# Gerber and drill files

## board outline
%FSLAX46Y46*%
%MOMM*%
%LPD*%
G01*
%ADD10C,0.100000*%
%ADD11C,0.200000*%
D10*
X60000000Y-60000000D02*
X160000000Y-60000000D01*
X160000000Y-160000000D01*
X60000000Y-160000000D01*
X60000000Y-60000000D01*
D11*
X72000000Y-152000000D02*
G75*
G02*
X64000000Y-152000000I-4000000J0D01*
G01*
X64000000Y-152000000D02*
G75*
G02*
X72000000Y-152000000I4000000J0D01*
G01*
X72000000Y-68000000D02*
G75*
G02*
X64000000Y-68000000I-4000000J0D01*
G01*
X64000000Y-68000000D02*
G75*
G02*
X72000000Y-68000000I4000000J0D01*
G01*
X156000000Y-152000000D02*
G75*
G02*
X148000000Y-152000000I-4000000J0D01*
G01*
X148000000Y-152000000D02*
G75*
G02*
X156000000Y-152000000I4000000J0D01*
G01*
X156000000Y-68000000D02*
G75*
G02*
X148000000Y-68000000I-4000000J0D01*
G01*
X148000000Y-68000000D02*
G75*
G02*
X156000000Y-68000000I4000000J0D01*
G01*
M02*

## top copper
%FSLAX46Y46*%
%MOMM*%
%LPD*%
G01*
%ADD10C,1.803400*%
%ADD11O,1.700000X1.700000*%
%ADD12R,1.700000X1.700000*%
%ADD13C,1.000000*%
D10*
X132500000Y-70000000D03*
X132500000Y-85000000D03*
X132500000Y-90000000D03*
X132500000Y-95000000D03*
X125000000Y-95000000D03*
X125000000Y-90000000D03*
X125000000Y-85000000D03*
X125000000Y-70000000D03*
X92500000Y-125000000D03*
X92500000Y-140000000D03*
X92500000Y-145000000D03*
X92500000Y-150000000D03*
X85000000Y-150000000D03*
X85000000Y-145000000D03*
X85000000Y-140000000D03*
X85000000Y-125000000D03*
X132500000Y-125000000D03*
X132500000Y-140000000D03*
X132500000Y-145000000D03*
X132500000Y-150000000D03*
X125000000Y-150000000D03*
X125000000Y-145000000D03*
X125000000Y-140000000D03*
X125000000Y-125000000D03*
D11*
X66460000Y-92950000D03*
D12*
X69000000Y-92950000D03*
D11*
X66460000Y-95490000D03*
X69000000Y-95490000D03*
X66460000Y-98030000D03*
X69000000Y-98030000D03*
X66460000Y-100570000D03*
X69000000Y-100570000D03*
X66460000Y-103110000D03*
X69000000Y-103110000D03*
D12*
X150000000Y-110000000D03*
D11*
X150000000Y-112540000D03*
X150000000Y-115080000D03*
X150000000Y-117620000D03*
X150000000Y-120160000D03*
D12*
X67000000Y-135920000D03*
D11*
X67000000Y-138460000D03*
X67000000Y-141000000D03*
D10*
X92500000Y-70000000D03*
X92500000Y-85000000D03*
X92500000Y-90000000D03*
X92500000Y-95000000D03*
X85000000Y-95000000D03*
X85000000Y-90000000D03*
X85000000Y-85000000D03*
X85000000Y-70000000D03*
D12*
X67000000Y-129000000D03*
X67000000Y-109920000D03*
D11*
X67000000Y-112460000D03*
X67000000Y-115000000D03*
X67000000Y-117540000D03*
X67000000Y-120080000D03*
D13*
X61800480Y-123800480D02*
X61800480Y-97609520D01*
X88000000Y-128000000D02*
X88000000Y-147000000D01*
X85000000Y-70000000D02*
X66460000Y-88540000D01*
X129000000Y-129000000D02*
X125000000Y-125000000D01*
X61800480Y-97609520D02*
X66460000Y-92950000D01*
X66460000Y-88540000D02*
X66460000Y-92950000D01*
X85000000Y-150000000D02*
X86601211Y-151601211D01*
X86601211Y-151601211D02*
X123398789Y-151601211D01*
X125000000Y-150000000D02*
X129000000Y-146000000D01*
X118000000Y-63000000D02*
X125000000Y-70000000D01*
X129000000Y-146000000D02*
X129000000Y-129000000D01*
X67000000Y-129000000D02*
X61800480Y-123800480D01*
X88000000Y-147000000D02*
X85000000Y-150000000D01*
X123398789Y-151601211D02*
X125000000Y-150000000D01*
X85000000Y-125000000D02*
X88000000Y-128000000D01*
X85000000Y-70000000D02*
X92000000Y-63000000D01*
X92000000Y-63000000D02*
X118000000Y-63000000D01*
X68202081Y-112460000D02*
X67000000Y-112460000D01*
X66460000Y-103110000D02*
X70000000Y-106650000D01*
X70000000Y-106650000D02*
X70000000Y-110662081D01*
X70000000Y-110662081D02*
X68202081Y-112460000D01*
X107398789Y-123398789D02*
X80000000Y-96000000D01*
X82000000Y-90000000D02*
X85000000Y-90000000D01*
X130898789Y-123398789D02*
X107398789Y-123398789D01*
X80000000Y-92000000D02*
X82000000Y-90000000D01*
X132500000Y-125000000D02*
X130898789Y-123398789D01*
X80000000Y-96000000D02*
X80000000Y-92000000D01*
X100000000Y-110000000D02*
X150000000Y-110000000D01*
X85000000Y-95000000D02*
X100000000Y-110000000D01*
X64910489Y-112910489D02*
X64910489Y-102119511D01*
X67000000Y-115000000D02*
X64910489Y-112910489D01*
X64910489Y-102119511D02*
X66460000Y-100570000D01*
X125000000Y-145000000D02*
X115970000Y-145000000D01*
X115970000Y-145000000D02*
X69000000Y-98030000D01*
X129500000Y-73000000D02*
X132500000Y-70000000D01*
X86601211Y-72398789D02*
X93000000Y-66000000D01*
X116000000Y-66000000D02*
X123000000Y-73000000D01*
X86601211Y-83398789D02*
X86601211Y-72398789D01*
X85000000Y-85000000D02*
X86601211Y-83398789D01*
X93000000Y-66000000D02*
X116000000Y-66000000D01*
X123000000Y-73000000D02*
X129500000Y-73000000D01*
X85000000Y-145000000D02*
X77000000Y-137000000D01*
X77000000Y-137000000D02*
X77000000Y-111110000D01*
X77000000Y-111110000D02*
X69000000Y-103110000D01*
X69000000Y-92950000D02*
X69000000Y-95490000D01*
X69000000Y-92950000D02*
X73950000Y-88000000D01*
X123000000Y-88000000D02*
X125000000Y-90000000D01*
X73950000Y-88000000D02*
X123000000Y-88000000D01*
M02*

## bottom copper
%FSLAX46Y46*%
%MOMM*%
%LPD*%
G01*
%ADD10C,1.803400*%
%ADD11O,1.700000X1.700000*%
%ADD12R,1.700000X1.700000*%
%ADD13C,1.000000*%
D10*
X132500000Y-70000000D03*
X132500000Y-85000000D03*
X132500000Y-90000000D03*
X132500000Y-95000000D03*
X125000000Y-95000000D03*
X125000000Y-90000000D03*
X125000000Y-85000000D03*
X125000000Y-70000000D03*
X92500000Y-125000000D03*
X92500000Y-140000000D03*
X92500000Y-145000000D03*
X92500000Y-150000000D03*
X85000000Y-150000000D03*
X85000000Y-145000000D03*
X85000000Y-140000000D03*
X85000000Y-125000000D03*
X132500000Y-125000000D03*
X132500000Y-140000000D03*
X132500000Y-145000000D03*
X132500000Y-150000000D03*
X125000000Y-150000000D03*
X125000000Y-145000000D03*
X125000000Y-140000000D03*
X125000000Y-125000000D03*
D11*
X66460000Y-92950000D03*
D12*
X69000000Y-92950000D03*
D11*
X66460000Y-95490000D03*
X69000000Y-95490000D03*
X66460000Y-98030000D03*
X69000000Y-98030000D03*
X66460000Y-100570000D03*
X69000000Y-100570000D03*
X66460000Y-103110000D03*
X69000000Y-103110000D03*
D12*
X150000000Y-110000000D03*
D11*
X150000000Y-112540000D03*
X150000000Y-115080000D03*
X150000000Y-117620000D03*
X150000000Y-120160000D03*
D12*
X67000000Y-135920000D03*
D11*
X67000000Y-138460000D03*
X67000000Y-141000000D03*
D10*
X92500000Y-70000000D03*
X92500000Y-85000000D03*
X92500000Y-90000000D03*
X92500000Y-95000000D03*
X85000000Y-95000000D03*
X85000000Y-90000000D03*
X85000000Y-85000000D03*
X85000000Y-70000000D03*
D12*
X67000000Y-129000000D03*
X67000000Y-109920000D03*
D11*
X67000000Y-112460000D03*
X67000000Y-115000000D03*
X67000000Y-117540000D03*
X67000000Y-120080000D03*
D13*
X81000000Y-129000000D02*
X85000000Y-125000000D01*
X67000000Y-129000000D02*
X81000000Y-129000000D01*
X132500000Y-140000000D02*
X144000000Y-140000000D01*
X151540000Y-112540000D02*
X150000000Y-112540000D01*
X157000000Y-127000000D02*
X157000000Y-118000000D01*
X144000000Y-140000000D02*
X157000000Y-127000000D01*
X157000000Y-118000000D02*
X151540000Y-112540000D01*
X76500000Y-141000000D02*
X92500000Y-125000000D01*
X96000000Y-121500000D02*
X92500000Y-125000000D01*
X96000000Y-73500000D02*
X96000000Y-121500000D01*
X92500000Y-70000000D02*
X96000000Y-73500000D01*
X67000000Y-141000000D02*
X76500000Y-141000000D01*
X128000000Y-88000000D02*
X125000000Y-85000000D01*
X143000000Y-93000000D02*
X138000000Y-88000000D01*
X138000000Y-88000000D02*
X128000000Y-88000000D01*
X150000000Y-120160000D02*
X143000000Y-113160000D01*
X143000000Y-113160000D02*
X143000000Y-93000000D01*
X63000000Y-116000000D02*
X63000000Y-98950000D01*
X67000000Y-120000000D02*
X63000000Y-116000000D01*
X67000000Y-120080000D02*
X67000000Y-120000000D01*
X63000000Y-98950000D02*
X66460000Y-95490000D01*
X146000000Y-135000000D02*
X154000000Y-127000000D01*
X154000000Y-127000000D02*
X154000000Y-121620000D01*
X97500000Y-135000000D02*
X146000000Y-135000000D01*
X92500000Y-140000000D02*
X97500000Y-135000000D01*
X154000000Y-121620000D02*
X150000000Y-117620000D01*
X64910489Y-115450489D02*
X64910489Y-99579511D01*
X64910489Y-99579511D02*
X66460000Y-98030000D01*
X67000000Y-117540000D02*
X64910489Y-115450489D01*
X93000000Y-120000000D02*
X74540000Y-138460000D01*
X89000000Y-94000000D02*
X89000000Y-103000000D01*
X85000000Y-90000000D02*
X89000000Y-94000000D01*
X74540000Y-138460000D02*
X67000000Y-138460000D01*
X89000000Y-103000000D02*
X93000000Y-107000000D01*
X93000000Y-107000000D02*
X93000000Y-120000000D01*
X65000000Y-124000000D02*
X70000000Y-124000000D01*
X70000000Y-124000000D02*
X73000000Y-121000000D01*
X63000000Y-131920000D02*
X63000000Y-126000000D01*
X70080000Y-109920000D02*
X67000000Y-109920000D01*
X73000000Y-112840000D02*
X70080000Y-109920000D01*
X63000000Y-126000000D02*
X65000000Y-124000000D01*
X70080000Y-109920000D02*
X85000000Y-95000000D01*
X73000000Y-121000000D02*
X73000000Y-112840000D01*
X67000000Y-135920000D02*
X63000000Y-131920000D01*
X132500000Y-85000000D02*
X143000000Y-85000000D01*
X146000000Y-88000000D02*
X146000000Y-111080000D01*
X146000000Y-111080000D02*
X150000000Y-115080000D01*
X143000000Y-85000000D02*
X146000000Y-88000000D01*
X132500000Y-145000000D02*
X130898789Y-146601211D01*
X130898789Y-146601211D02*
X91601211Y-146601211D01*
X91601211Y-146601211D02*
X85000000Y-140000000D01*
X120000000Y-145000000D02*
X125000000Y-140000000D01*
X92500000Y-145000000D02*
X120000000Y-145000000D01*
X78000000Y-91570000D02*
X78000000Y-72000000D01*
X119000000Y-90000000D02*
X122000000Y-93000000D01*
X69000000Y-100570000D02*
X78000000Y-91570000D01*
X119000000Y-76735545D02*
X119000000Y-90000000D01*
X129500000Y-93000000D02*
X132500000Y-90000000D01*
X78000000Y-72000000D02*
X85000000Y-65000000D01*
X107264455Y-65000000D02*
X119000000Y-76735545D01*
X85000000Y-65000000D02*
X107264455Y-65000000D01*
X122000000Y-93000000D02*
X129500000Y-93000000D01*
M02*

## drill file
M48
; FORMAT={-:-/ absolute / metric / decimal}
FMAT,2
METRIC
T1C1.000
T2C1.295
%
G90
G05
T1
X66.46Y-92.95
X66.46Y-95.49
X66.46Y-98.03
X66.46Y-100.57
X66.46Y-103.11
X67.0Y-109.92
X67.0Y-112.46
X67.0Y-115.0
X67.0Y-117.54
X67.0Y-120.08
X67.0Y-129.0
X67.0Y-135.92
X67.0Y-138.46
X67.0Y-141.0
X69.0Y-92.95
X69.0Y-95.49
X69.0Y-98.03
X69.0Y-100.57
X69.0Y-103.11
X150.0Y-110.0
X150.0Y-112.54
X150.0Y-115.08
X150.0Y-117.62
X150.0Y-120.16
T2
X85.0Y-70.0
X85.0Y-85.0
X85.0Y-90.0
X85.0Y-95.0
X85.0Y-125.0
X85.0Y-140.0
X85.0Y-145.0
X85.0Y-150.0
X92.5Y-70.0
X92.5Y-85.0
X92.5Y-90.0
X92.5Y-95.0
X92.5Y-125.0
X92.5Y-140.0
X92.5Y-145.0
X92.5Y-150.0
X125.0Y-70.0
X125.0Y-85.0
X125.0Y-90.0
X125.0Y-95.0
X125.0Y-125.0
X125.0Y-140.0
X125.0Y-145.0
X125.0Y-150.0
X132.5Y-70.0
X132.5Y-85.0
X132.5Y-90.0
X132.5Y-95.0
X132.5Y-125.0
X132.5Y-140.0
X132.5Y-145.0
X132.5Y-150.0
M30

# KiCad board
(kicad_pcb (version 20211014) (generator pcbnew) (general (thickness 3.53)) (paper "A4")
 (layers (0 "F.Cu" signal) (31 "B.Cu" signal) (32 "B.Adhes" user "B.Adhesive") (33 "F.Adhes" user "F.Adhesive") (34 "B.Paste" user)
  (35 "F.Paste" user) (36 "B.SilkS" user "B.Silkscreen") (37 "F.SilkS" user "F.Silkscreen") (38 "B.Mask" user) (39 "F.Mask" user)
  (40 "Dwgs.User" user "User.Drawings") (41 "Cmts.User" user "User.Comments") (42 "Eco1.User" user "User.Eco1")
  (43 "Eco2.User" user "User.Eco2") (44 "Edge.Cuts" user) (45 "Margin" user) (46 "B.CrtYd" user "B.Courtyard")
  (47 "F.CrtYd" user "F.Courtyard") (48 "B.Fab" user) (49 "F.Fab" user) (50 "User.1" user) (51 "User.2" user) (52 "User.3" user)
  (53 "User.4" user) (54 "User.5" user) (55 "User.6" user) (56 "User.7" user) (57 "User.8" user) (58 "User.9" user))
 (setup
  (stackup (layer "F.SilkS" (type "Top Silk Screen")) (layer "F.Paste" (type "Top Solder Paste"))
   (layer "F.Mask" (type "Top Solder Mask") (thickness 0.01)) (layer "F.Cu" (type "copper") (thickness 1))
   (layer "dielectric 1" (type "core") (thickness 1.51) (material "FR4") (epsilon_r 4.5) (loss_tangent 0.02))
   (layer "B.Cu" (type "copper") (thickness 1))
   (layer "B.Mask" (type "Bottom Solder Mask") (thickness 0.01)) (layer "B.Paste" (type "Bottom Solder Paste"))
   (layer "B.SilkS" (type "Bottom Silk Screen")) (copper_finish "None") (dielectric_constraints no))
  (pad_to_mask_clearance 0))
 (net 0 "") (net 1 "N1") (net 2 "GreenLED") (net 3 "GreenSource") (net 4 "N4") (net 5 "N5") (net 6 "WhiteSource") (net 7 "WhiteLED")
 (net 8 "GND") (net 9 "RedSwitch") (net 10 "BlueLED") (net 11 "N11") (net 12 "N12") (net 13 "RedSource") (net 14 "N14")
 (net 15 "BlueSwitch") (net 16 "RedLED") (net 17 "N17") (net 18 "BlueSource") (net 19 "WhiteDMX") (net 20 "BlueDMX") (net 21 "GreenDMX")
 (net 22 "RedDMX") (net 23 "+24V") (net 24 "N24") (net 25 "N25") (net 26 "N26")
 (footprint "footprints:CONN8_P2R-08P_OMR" (layer "F.Cu") (at 125 70)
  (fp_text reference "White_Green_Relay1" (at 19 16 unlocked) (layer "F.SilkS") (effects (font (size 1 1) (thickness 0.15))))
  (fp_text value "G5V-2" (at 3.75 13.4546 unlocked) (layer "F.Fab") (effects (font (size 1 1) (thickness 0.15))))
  (pad "1" thru_hole circle (at 7.5 0) (size 1.8034 1.8034) (drill 1.2954) (layers *.Cu *.Mask) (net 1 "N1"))
  (pad "4" thru_hole circle (at 7.5 15) (size 1.8034 1.8034) (drill 1.2954) (layers *.Cu *.Mask) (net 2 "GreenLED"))
  (pad "6" thru_hole circle (at 7.5 20) (size 1.8034 1.8034) (drill 1.2954) (layers *.Cu *.Mask) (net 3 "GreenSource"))
  (pad "8" thru_hole circle (at 7.5 25) (size 1.8034 1.8034) (drill 1.2954) (layers *.Cu *.Mask) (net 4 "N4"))
  (pad "9" thru_hole circle (at 0 25) (size 1.8034 1.8034) (drill 1.2954) (layers *.Cu *.Mask) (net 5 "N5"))
  (pad "11" thru_hole circle (at 0 20) (size 1.8034 1.8034) (drill 1.2954) (layers *.Cu *.Mask) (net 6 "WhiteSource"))
  (pad "13" thru_hole circle (at 0 15) (size 1.8034 1.8034) (drill 1.2954) (layers *.Cu *.Mask) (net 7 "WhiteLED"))
  (pad "16" thru_hole circle (at 0 0) (size 1.8034 1.8034) (drill 1.2954) (layers *.Cu *.Mask) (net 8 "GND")))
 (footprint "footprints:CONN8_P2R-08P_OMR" (layer "F.Cu") (at 85 125)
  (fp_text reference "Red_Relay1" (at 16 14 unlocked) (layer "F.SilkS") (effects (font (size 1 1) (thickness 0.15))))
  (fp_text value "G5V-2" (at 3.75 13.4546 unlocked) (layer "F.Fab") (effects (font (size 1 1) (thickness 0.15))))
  (pad "1" thru_hole circle (at 7.5 0) (size 1.8034 1.8034) (drill 1.2954) (layers *.Cu *.Mask) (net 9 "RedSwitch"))
  (pad "4" thru_hole circle (at 7.5 15) (size 1.8034 1.8034) (drill 1.2954) (layers *.Cu *.Mask) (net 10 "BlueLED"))
  (pad "6" thru_hole circle (at 7.5 20) (size 1.8034 1.8034) (drill 1.2954) (layers *.Cu *.Mask) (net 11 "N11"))
  (pad "8" thru_hole circle (at 7.5 25) (size 1.8034 1.8034) (drill 1.2954) (layers *.Cu *.Mask) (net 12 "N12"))
  (pad "9" thru_hole circle (at 0 25) (size 1.8034 1.8034) (drill 1.2954) (layers *.Cu *.Mask) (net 8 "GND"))
  (pad "11" thru_hole circle (at 0 20) (size 1.8034 1.8034) (drill 1.2954) (layers *.Cu *.Mask) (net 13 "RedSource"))
  (pad "13" thru_hole circle (at 0 15) (size 1.8034 1.8034) (drill 1.2954) (layers *.Cu *.Mask) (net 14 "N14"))
  (pad "16" thru_hole circle (at 0 0) (size 1.8034 1.8034) (drill 1.2954) (layers *.Cu *.Mask) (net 8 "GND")))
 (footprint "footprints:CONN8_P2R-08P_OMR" (layer "F.Cu") (at 125 125)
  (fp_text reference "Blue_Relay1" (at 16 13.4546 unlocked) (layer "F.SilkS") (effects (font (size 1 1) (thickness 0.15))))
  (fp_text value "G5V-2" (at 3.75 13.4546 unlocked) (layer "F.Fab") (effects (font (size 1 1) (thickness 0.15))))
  (pad "1" thru_hole circle (at 7.5 0) (size 1.8034 1.8034) (drill 1.2954) (layers *.Cu *.Mask) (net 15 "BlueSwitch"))
  (pad "4" thru_hole circle (at 7.5 15) (size 1.8034 1.8034) (drill 1.2954) (layers *.Cu *.Mask) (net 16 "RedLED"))
  (pad "6" thru_hole circle (at 7.5 20) (size 1.8034 1.8034) (drill 1.2954) (layers *.Cu *.Mask) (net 14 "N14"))
  (pad "8" thru_hole circle (at 7.5 25) (size 1.8034 1.8034) (drill 1.2954) (layers *.Cu *.Mask) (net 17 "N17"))
  (pad "9" thru_hole circle (at 0 25) (size 1.8034 1.8034) (drill 1.2954) (layers *.Cu *.Mask) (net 8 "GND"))
  (pad "11" thru_hole circle (at 0 20) (size 1.8034 1.8034) (drill 1.2954) (layers *.Cu *.Mask) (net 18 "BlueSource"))
  (pad "13" thru_hole circle (at 0 15) (size 1.8034 1.8034) (drill 1.2954) (layers *.Cu *.Mask) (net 11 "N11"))
  (pad "16" thru_hole circle (at 0 0) (size 1.8034 1.8034) (drill 1.2954) (layers *.Cu *.Mask) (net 8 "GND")))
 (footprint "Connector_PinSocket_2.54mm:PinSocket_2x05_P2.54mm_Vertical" (layer "F.Cu") (at 69 92.95)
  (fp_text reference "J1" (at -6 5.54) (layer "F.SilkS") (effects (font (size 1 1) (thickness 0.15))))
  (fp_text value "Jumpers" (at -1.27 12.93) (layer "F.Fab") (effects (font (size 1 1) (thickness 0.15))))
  (pad "1a" thru_hole oval (at -2.54 0) (size 1.7 1.7) (drill 1) (layers *.Cu *.Mask) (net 8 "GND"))
  (pad "1b" thru_hole rect (at 0 0) (size 1.7 1.7) (drill 1) (layers *.Cu *.Mask) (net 6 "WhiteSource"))
  (pad "2a" thru_hole oval (at -2.54 2.54) (size 1.7 1.7) (drill 1) (layers *.Cu *.Mask) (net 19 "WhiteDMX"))
  (pad "2b" thru_hole oval (at 0 2.54) (size 1.7 1.7) (drill 1) (layers *.Cu *.Mask) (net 6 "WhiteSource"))
  (pad "3a" thru_hole oval (at -2.54 5.08) (size 1.7 1.7) (drill 1) (layers *.Cu *.Mask) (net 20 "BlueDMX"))
  (pad "3b" thru_hole oval (at 0 5.08) (size 1.7 1.7) (drill 1) (layers *.Cu *.Mask) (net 18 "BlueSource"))
  (pad "4a" thru_hole oval (at -2.54 7.62) (size 1.7 1.7) (drill 1) (layers *.Cu *.Mask) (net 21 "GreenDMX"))
  (pad "4b" thru_hole oval (at 0 7.62) (size 1.7 1.7) (drill 1) (layers *.Cu *.Mask) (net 3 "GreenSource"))
  (pad "5a" thru_hole oval (at -2.54 10.16) (size 1.7 1.7) (drill 1) (layers *.Cu *.Mask) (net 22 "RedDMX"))
  (pad "5b" thru_hole oval (at 0 10.16) (size 1.7 1.7) (drill 1) (layers *.Cu *.Mask) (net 13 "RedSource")))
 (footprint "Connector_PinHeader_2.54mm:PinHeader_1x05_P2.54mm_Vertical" (layer "F.Cu") (at 150 110)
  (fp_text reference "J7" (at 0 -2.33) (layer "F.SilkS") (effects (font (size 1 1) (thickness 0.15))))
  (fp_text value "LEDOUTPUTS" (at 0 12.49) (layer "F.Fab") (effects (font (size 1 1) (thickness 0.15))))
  (pad "1" thru_hole rect (at 0 0) (size 1.7 1.7) (drill 1) (layers *.Cu *.Mask) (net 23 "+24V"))
  (pad "2" thru_hole oval (at 0 2.54) (size 1.7 1.7) (drill 1) (layers *.Cu *.Mask) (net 16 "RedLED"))
  (pad "3" thru_hole oval (at 0 5.08) (size 1.7 1.7) (drill 1) (layers *.Cu *.Mask) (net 2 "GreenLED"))
  (pad "4" thru_hole oval (at 0 7.62) (size 1.7 1.7) (drill 1) (layers *.Cu *.Mask) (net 10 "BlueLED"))
  (pad "5" thru_hole oval (at 0 10.16) (size 1.7 1.7) (drill 1) (layers *.Cu *.Mask) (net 7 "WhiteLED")))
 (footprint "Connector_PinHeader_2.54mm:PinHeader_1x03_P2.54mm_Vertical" (layer "F.Cu") (at 67 135.92)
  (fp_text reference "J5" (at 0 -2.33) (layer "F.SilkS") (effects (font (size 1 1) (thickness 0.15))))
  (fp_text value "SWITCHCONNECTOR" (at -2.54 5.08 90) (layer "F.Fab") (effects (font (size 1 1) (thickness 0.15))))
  (pad "1" thru_hole rect (at 0 0) (size 1.7 1.7) (drill 1) (layers *.Cu *.Mask) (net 23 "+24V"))
  (pad "2" thru_hole oval (at 0 2.54) (size 1.7 1.7) (drill 1) (layers *.Cu *.Mask) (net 15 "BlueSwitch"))
  (pad "3" thru_hole oval (at 0 5.08) (size 1.7 1.7) (drill 1) (layers *.Cu *.Mask) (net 9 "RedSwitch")))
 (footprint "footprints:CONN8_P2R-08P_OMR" (layer "F.Cu") (at 85 70)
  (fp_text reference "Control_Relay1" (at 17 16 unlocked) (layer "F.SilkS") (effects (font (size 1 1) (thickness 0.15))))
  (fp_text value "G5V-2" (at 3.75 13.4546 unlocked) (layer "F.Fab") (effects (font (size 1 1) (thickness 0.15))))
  (pad "1" thru_hole circle (at 7.5 0) (size 1.8034 1.8034) (drill 1.2954) (layers *.Cu *.Mask) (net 9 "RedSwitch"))
  (pad "4" thru_hole circle (at 7.5 15) (size 1.8034 1.8034) (drill 1.2954) (layers *.Cu *.Mask) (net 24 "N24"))
  (pad "6" thru_hole circle (at 7.5 20) (size 1.8034 1.8034) (drill 1.2954) (layers *.Cu *.Mask) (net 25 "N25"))
  (pad "8" thru_hole circle (at 7.5 25) (size 1.8034 1.8034) (drill 1.2954) (layers *.Cu *.Mask) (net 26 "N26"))
  (pad "9" thru_hole circle (at 0 25) (size 1.8034 1.8034) (drill 1.2954) (layers *.Cu *.Mask) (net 23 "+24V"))
  (pad "11" thru_hole circle (at 0 20) (size 1.8034 1.8034) (drill 1.2954) (layers *.Cu *.Mask) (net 15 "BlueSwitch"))
  (pad "13" thru_hole circle (at 0 15) (size 1.8034 1.8034) (drill 1.2954) (layers *.Cu *.Mask) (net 1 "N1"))
  (pad "16" thru_hole circle (at 0 0) (size 1.8034 1.8034) (drill 1.2954) (layers *.Cu *.Mask) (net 8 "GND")))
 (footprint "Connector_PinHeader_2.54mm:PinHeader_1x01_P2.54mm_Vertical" (layer "F.Cu") (at 67 129)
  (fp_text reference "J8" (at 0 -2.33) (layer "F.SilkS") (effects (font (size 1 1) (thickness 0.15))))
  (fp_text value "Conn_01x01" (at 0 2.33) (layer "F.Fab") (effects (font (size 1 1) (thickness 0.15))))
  (pad "1" thru_hole rect (at 0 0) (size 1.7 1.7) (drill 1) (layers *.Cu *.Mask) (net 8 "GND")))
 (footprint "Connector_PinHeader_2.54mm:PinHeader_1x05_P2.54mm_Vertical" (layer "F.Cu") (at 67 109.92)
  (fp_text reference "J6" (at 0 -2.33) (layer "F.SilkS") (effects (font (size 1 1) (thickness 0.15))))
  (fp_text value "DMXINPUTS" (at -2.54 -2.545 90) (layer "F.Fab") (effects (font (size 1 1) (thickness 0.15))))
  (pad "1" thru_hole rect (at 0 0) (size 1.7 1.7) (drill 1) (layers *.Cu *.Mask) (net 23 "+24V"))
  (pad "2" thru_hole oval (at 0 2.54) (size 1.7 1.7) (drill 1) (layers *.Cu *.Mask) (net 22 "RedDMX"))
  (pad "3" thru_hole oval (at 0 5.08) (size 1.7 1.7) (drill 1) (layers *.Cu *.Mask) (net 21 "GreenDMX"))
  (pad "4" thru_hole oval (at 0 7.62) (size 1.7 1.7) (drill 1) (layers *.Cu *.Mask) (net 20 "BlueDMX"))
  (pad "5" thru_hole oval (at 0 10.16) (size 1.7 1.7) (drill 1) (layers *.Cu *.Mask) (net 19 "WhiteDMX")))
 (gr_rect (start 60 60) (end 160 160) (layer "Edge.Cuts") (width 0.1) (fill none))
 (gr_circle (center 68 152) (end 72 152) (layer "Edge.Cuts") (width 0.2) (fill none))
 (gr_circle (center 68 68) (end 72 68) (layer "Edge.Cuts") (width 0.2) (fill none))
 (gr_circle (center 152 152) (end 156 152) (layer "Edge.Cuts") (width 0.2) (fill none))
 (gr_circle (center 152 68) (end 156 68) (layer "Edge.Cuts") (width 0.2) (fill none))
 (segment (start 61.80048 123.80048) (end 61.80048 97.60952) (width 1) (layer "F.Cu") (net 8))
 (segment (start 88 128) (end 88 147) (width 1) (layer "F.Cu") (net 8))
 (segment (start 85 70) (end 66.46 88.54) (width 1) (layer "F.Cu") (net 8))
 (segment (start 129 129) (end 125 125) (width 1) (layer "F.Cu") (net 8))
 (segment (start 61.80048 97.60952) (end 66.46 92.95) (width 1) (layer "F.Cu") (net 8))
 (segment (start 66.46 88.54) (end 66.46 92.95) (width 1) (layer "F.Cu") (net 8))
 (segment (start 85 150) (end 86.601211 151.601211) (width 1) (layer "F.Cu") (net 8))
 (segment (start 86.601211 151.601211) (end 123.398789 151.601211) (width 1) (layer "F.Cu") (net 8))
 (segment (start 125 150) (end 129 146) (width 1) (layer "F.Cu") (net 8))
 (segment (start 118 63) (end 125 70) (width 1) (layer "F.Cu") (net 8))
 (segment (start 129 146) (end 129 129) (width 1) (layer "F.Cu") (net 8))
 (segment (start 67 129) (end 61.80048 123.80048) (width 1) (layer "F.Cu") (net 8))
 (segment (start 88 147) (end 85 150) (width 1) (layer "F.Cu") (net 8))
 (segment (start 123.398789 151.601211) (end 125 150) (width 1) (layer "F.Cu") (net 8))
 (segment (start 85 125) (end 88 128) (width 1) (layer "F.Cu") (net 8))
 (segment (start 85 70) (end 92 63) (width 1) (layer "F.Cu") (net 8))
 (segment (start 92 63) (end 118 63) (width 1) (layer "F.Cu") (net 8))
 (segment (start 81 129) (end 85 125) (width 1) (layer "B.Cu") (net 8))
 (segment (start 67 129) (end 81 129) (width 1) (layer "B.Cu") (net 8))
 (segment (start 132.5 140) (end 144 140) (width 1) (layer "B.Cu") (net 16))
 (segment (start 151.54 112.54) (end 150 112.54) (width 1) (layer "B.Cu") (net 16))
 (segment (start 157 127) (end 157 118) (width 1) (layer "B.Cu") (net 16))
 (segment (start 144 140) (end 157 127) (width 1) (layer "B.Cu") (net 16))
 (segment (start 157 118) (end 151.54 112.54) (width 1) (layer "B.Cu") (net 16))
 (segment (start 68.202081 112.46) (end 67 112.46) (width 1) (layer "F.Cu") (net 22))
 (segment (start 66.46 103.11) (end 70 106.65) (width 1) (layer "F.Cu") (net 22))
 (segment (start 70 106.65) (end 70 110.662081) (width 1) (layer "F.Cu") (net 22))
 (segment (start 70 110.662081) (end 68.202081 112.46) (width 1) (layer "F.Cu") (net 22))
 (segment (start 76.5 141) (end 92.5 125) (width 1) (layer "B.Cu") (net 9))
 (segment (start 96 121.5) (end 92.5 125) (width 1) (layer "B.Cu") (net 9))
 (segment (start 96 73.5) (end 96 121.5) (width 1) (layer "B.Cu") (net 9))
 (segment (start 92.5 70) (end 96 73.5) (width 1) (layer "B.Cu") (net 9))
 (segment (start 67 141) (end 76.5 141) (width 1) (layer "B.Cu") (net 9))
 (segment (start 128 88) (end 125 85) (width 1) (layer "B.Cu") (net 7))
 (segment (start 143 93) (end 138 88) (width 1) (layer "B.Cu") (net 7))
 (segment (start 138 88) (end 128 88) (width 1) (layer "B.Cu") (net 7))
 (segment (start 150 120.16) (end 143 113.16) (width 1) (layer "B.Cu") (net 7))
 (segment (start 143 113.16) (end 143 93) (width 1) (layer "B.Cu") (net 7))
 (segment (start 63 116) (end 63 98.95) (width 1) (layer "B.Cu") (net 19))
 (segment (start 67 120) (end 63 116) (width 1) (layer "B.Cu") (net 19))
 (segment (start 67 120.08) (end 67 120) (width 1) (layer "B.Cu") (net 19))
 (segment (start 63 98.95) (end 66.46 95.49) (width 1) (layer "B.Cu") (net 19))
 (segment (start 146 135) (end 154 127) (width 1) (layer "B.Cu") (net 10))
 (segment (start 154 127) (end 154 121.62) (width 1) (layer "B.Cu") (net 10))
 (segment (start 97.5 135) (end 146 135) (width 1) (layer "B.Cu") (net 10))
 (segment (start 92.5 140) (end 97.5 135) (width 1) (layer "B.Cu") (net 10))
 (segment (start 154 121.62) (end 150 117.62) (width 1) (layer "B.Cu") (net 10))
 (segment (start 64.910489 115.450489) (end 64.910489 99.579511) (width 1) (layer "B.Cu") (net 20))
 (segment (start 64.910489 99.579511) (end 66.46 98.03) (width 1) (layer "B.Cu") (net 20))
 (segment (start 67 117.54) (end 64.910489 115.450489) (width 1) (layer "B.Cu") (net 20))
 (segment (start 107.398789 123.398789) (end 80 96) (width 1) (layer "F.Cu") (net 15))
 (segment (start 82 90) (end 85 90) (width 1) (layer "F.Cu") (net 15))
 (segment (start 130.898789 123.398789) (end 107.398789 123.398789) (width 1) (layer "F.Cu") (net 15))
 (segment (start 80 92) (end 82 90) (width 1) (layer "F.Cu") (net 15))
 (segment (start 132.5 125) (end 130.898789 123.398789) (width 1) (layer "F.Cu") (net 15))
 (segment (start 80 96) (end 80 92) (width 1) (layer "F.Cu") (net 15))
 (segment (start 93 120) (end 74.54 138.46) (width 1) (layer "B.Cu") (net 15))
 (segment (start 89 94) (end 89 103) (width 1) (layer "B.Cu") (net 15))
 (segment (start 85 90) (end 89 94) (width 1) (layer "B.Cu") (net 15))
 (segment (start 74.54 138.46) (end 67 138.46) (width 1) (layer "B.Cu") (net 15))
 (segment (start 89 103) (end 93 107) (width 1) (layer "B.Cu") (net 15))
 (segment (start 93 107) (end 93 120) (width 1) (layer "B.Cu") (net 15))
 (segment (start 100 110) (end 150 110) (width 1) (layer "F.Cu") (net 23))
 (segment (start 85 95) (end 100 110) (width 1) (layer "F.Cu") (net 23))
 (segment (start 65 124) (end 70 124) (width 1) (layer "B.Cu") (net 23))
 (segment (start 70 124) (end 73 121) (width 1) (layer "B.Cu") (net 23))
 (segment (start 63 131.92) (end 63 126) (width 1) (layer "B.Cu") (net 23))
 (segment (start 70.08 109.92) (end 67 109.92) (width 1) (layer "B.Cu") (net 23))
 (segment (start 73 112.84) (end 70.08 109.92) (width 1) (layer "B.Cu") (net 23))
 (segment (start 63 126) (end 65 124) (width 1) (layer "B.Cu") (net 23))
 (segment (start 70.08 109.92) (end 85 95) (width 1) (layer "B.Cu") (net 23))
 (segment (start 73 121) (end 73 112.84) (width 1) (layer "B.Cu") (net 23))
 (segment (start 67 135.92) (end 63 131.92) (width 1) (layer "B.Cu") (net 23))
 (segment (start 64.910489 112.910489) (end 64.910489 102.119511) (width 1) (layer "F.Cu") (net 21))
 (segment (start 67 115) (end 64.910489 112.910489) (width 1) (layer "F.Cu") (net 21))
 (segment (start 64.910489 102.119511) (end 66.46 100.57) (width 1) (layer "F.Cu") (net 21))
 (segment (start 132.5 85) (end 143 85) (width 1) (layer "B.Cu") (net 2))
 (segment (start 146 88) (end 146 111.08) (width 1) (layer "B.Cu") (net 2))
 (segment (start 146 111.08) (end 150 115.08) (width 1) (layer "B.Cu") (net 2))
 (segment (start 143 85) (end 146 88) (width 1) (layer "B.Cu") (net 2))
 (segment (start 132.5 145) (end 130.898789 146.601211) (width 1) (layer "B.Cu") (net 14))
 (segment (start 130.898789 146.601211) (end 91.601211 146.601211) (width 1) (layer "B.Cu") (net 14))
 (segment (start 91.601211 146.601211) (end 85 140) (width 1) (layer "B.Cu") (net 14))
 (segment (start 125 145) (end 115.97 145) (width 1) (layer "F.Cu") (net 18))
 (segment (start 115.97 145) (end 69 98.03) (width 1) (layer "F.Cu") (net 18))
 (segment (start 120 145) (end 125 140) (width 1) (layer "B.Cu") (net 11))
 (segment (start 92.5 145) (end 120 145) (width 1) (layer "B.Cu") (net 11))
 (segment (start 129.5 73) (end 132.5 70) (width 1) (layer "F.Cu") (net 1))
 (segment (start 86.601211 72.398789) (end 93 66) (width 1) (layer "F.Cu") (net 1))
 (segment (start 116 66) (end 123 73) (width 1) (layer "F.Cu") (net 1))
 (segment (start 86.601211 83.398789) (end 86.601211 72.398789) (width 1) (layer "F.Cu") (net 1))
 (segment (start 85 85) (end 86.601211 83.398789) (width 1) (layer "F.Cu") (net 1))
 (segment (start 93 66) (end 116 66) (width 1) (layer "F.Cu") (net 1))
 (segment (start 123 73) (end 129.5 73) (width 1) (layer "F.Cu") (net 1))
 (segment (start 85 145) (end 77 137) (width 1) (layer "F.Cu") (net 13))
 (segment (start 77 137) (end 77 111.11) (width 1) (layer "F.Cu") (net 13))
 (segment (start 77 111.11) (end 69 103.11) (width 1) (layer "F.Cu") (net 13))
 (segment (start 78 91.57) (end 78 72) (width 1) (layer "B.Cu") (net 3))
 (segment (start 119 90) (end 122 93) (width 1) (layer "B.Cu") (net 3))
 (segment (start 69 100.57) (end 78 91.57) (width 1) (layer "B.Cu") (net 3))
 (segment (start 119 76.735545) (end 119 90) (width 1) (layer "B.Cu") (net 3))
 (segment (start 129.5 93) (end 132.5 90) (width 1) (layer "B.Cu") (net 3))
 (segment (start 78 72) (end 85 65) (width 1) (layer "B.Cu") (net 3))
 (segment (start 107.264455 65) (end 119 76.735545) (width 1) (layer "B.Cu") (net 3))
 (segment (start 85 65) (end 107.264455 65) (width 1) (layer "B.Cu") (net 3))
 (segment (start 122 93) (end 129.5 93) (width 1) (layer "B.Cu") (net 3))
 (segment (start 69 92.95) (end 69 95.49) (width 1) (layer "F.Cu") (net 6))
 (segment (start 69 92.95) (end 73.95 88) (width 1) (layer "F.Cu") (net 6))
 (segment (start 123 88) (end 125 90) (width 1) (layer "F.Cu") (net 6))
 (segment (start 73.95 88) (end 123 88) (width 1) (layer "F.Cu") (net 6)))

